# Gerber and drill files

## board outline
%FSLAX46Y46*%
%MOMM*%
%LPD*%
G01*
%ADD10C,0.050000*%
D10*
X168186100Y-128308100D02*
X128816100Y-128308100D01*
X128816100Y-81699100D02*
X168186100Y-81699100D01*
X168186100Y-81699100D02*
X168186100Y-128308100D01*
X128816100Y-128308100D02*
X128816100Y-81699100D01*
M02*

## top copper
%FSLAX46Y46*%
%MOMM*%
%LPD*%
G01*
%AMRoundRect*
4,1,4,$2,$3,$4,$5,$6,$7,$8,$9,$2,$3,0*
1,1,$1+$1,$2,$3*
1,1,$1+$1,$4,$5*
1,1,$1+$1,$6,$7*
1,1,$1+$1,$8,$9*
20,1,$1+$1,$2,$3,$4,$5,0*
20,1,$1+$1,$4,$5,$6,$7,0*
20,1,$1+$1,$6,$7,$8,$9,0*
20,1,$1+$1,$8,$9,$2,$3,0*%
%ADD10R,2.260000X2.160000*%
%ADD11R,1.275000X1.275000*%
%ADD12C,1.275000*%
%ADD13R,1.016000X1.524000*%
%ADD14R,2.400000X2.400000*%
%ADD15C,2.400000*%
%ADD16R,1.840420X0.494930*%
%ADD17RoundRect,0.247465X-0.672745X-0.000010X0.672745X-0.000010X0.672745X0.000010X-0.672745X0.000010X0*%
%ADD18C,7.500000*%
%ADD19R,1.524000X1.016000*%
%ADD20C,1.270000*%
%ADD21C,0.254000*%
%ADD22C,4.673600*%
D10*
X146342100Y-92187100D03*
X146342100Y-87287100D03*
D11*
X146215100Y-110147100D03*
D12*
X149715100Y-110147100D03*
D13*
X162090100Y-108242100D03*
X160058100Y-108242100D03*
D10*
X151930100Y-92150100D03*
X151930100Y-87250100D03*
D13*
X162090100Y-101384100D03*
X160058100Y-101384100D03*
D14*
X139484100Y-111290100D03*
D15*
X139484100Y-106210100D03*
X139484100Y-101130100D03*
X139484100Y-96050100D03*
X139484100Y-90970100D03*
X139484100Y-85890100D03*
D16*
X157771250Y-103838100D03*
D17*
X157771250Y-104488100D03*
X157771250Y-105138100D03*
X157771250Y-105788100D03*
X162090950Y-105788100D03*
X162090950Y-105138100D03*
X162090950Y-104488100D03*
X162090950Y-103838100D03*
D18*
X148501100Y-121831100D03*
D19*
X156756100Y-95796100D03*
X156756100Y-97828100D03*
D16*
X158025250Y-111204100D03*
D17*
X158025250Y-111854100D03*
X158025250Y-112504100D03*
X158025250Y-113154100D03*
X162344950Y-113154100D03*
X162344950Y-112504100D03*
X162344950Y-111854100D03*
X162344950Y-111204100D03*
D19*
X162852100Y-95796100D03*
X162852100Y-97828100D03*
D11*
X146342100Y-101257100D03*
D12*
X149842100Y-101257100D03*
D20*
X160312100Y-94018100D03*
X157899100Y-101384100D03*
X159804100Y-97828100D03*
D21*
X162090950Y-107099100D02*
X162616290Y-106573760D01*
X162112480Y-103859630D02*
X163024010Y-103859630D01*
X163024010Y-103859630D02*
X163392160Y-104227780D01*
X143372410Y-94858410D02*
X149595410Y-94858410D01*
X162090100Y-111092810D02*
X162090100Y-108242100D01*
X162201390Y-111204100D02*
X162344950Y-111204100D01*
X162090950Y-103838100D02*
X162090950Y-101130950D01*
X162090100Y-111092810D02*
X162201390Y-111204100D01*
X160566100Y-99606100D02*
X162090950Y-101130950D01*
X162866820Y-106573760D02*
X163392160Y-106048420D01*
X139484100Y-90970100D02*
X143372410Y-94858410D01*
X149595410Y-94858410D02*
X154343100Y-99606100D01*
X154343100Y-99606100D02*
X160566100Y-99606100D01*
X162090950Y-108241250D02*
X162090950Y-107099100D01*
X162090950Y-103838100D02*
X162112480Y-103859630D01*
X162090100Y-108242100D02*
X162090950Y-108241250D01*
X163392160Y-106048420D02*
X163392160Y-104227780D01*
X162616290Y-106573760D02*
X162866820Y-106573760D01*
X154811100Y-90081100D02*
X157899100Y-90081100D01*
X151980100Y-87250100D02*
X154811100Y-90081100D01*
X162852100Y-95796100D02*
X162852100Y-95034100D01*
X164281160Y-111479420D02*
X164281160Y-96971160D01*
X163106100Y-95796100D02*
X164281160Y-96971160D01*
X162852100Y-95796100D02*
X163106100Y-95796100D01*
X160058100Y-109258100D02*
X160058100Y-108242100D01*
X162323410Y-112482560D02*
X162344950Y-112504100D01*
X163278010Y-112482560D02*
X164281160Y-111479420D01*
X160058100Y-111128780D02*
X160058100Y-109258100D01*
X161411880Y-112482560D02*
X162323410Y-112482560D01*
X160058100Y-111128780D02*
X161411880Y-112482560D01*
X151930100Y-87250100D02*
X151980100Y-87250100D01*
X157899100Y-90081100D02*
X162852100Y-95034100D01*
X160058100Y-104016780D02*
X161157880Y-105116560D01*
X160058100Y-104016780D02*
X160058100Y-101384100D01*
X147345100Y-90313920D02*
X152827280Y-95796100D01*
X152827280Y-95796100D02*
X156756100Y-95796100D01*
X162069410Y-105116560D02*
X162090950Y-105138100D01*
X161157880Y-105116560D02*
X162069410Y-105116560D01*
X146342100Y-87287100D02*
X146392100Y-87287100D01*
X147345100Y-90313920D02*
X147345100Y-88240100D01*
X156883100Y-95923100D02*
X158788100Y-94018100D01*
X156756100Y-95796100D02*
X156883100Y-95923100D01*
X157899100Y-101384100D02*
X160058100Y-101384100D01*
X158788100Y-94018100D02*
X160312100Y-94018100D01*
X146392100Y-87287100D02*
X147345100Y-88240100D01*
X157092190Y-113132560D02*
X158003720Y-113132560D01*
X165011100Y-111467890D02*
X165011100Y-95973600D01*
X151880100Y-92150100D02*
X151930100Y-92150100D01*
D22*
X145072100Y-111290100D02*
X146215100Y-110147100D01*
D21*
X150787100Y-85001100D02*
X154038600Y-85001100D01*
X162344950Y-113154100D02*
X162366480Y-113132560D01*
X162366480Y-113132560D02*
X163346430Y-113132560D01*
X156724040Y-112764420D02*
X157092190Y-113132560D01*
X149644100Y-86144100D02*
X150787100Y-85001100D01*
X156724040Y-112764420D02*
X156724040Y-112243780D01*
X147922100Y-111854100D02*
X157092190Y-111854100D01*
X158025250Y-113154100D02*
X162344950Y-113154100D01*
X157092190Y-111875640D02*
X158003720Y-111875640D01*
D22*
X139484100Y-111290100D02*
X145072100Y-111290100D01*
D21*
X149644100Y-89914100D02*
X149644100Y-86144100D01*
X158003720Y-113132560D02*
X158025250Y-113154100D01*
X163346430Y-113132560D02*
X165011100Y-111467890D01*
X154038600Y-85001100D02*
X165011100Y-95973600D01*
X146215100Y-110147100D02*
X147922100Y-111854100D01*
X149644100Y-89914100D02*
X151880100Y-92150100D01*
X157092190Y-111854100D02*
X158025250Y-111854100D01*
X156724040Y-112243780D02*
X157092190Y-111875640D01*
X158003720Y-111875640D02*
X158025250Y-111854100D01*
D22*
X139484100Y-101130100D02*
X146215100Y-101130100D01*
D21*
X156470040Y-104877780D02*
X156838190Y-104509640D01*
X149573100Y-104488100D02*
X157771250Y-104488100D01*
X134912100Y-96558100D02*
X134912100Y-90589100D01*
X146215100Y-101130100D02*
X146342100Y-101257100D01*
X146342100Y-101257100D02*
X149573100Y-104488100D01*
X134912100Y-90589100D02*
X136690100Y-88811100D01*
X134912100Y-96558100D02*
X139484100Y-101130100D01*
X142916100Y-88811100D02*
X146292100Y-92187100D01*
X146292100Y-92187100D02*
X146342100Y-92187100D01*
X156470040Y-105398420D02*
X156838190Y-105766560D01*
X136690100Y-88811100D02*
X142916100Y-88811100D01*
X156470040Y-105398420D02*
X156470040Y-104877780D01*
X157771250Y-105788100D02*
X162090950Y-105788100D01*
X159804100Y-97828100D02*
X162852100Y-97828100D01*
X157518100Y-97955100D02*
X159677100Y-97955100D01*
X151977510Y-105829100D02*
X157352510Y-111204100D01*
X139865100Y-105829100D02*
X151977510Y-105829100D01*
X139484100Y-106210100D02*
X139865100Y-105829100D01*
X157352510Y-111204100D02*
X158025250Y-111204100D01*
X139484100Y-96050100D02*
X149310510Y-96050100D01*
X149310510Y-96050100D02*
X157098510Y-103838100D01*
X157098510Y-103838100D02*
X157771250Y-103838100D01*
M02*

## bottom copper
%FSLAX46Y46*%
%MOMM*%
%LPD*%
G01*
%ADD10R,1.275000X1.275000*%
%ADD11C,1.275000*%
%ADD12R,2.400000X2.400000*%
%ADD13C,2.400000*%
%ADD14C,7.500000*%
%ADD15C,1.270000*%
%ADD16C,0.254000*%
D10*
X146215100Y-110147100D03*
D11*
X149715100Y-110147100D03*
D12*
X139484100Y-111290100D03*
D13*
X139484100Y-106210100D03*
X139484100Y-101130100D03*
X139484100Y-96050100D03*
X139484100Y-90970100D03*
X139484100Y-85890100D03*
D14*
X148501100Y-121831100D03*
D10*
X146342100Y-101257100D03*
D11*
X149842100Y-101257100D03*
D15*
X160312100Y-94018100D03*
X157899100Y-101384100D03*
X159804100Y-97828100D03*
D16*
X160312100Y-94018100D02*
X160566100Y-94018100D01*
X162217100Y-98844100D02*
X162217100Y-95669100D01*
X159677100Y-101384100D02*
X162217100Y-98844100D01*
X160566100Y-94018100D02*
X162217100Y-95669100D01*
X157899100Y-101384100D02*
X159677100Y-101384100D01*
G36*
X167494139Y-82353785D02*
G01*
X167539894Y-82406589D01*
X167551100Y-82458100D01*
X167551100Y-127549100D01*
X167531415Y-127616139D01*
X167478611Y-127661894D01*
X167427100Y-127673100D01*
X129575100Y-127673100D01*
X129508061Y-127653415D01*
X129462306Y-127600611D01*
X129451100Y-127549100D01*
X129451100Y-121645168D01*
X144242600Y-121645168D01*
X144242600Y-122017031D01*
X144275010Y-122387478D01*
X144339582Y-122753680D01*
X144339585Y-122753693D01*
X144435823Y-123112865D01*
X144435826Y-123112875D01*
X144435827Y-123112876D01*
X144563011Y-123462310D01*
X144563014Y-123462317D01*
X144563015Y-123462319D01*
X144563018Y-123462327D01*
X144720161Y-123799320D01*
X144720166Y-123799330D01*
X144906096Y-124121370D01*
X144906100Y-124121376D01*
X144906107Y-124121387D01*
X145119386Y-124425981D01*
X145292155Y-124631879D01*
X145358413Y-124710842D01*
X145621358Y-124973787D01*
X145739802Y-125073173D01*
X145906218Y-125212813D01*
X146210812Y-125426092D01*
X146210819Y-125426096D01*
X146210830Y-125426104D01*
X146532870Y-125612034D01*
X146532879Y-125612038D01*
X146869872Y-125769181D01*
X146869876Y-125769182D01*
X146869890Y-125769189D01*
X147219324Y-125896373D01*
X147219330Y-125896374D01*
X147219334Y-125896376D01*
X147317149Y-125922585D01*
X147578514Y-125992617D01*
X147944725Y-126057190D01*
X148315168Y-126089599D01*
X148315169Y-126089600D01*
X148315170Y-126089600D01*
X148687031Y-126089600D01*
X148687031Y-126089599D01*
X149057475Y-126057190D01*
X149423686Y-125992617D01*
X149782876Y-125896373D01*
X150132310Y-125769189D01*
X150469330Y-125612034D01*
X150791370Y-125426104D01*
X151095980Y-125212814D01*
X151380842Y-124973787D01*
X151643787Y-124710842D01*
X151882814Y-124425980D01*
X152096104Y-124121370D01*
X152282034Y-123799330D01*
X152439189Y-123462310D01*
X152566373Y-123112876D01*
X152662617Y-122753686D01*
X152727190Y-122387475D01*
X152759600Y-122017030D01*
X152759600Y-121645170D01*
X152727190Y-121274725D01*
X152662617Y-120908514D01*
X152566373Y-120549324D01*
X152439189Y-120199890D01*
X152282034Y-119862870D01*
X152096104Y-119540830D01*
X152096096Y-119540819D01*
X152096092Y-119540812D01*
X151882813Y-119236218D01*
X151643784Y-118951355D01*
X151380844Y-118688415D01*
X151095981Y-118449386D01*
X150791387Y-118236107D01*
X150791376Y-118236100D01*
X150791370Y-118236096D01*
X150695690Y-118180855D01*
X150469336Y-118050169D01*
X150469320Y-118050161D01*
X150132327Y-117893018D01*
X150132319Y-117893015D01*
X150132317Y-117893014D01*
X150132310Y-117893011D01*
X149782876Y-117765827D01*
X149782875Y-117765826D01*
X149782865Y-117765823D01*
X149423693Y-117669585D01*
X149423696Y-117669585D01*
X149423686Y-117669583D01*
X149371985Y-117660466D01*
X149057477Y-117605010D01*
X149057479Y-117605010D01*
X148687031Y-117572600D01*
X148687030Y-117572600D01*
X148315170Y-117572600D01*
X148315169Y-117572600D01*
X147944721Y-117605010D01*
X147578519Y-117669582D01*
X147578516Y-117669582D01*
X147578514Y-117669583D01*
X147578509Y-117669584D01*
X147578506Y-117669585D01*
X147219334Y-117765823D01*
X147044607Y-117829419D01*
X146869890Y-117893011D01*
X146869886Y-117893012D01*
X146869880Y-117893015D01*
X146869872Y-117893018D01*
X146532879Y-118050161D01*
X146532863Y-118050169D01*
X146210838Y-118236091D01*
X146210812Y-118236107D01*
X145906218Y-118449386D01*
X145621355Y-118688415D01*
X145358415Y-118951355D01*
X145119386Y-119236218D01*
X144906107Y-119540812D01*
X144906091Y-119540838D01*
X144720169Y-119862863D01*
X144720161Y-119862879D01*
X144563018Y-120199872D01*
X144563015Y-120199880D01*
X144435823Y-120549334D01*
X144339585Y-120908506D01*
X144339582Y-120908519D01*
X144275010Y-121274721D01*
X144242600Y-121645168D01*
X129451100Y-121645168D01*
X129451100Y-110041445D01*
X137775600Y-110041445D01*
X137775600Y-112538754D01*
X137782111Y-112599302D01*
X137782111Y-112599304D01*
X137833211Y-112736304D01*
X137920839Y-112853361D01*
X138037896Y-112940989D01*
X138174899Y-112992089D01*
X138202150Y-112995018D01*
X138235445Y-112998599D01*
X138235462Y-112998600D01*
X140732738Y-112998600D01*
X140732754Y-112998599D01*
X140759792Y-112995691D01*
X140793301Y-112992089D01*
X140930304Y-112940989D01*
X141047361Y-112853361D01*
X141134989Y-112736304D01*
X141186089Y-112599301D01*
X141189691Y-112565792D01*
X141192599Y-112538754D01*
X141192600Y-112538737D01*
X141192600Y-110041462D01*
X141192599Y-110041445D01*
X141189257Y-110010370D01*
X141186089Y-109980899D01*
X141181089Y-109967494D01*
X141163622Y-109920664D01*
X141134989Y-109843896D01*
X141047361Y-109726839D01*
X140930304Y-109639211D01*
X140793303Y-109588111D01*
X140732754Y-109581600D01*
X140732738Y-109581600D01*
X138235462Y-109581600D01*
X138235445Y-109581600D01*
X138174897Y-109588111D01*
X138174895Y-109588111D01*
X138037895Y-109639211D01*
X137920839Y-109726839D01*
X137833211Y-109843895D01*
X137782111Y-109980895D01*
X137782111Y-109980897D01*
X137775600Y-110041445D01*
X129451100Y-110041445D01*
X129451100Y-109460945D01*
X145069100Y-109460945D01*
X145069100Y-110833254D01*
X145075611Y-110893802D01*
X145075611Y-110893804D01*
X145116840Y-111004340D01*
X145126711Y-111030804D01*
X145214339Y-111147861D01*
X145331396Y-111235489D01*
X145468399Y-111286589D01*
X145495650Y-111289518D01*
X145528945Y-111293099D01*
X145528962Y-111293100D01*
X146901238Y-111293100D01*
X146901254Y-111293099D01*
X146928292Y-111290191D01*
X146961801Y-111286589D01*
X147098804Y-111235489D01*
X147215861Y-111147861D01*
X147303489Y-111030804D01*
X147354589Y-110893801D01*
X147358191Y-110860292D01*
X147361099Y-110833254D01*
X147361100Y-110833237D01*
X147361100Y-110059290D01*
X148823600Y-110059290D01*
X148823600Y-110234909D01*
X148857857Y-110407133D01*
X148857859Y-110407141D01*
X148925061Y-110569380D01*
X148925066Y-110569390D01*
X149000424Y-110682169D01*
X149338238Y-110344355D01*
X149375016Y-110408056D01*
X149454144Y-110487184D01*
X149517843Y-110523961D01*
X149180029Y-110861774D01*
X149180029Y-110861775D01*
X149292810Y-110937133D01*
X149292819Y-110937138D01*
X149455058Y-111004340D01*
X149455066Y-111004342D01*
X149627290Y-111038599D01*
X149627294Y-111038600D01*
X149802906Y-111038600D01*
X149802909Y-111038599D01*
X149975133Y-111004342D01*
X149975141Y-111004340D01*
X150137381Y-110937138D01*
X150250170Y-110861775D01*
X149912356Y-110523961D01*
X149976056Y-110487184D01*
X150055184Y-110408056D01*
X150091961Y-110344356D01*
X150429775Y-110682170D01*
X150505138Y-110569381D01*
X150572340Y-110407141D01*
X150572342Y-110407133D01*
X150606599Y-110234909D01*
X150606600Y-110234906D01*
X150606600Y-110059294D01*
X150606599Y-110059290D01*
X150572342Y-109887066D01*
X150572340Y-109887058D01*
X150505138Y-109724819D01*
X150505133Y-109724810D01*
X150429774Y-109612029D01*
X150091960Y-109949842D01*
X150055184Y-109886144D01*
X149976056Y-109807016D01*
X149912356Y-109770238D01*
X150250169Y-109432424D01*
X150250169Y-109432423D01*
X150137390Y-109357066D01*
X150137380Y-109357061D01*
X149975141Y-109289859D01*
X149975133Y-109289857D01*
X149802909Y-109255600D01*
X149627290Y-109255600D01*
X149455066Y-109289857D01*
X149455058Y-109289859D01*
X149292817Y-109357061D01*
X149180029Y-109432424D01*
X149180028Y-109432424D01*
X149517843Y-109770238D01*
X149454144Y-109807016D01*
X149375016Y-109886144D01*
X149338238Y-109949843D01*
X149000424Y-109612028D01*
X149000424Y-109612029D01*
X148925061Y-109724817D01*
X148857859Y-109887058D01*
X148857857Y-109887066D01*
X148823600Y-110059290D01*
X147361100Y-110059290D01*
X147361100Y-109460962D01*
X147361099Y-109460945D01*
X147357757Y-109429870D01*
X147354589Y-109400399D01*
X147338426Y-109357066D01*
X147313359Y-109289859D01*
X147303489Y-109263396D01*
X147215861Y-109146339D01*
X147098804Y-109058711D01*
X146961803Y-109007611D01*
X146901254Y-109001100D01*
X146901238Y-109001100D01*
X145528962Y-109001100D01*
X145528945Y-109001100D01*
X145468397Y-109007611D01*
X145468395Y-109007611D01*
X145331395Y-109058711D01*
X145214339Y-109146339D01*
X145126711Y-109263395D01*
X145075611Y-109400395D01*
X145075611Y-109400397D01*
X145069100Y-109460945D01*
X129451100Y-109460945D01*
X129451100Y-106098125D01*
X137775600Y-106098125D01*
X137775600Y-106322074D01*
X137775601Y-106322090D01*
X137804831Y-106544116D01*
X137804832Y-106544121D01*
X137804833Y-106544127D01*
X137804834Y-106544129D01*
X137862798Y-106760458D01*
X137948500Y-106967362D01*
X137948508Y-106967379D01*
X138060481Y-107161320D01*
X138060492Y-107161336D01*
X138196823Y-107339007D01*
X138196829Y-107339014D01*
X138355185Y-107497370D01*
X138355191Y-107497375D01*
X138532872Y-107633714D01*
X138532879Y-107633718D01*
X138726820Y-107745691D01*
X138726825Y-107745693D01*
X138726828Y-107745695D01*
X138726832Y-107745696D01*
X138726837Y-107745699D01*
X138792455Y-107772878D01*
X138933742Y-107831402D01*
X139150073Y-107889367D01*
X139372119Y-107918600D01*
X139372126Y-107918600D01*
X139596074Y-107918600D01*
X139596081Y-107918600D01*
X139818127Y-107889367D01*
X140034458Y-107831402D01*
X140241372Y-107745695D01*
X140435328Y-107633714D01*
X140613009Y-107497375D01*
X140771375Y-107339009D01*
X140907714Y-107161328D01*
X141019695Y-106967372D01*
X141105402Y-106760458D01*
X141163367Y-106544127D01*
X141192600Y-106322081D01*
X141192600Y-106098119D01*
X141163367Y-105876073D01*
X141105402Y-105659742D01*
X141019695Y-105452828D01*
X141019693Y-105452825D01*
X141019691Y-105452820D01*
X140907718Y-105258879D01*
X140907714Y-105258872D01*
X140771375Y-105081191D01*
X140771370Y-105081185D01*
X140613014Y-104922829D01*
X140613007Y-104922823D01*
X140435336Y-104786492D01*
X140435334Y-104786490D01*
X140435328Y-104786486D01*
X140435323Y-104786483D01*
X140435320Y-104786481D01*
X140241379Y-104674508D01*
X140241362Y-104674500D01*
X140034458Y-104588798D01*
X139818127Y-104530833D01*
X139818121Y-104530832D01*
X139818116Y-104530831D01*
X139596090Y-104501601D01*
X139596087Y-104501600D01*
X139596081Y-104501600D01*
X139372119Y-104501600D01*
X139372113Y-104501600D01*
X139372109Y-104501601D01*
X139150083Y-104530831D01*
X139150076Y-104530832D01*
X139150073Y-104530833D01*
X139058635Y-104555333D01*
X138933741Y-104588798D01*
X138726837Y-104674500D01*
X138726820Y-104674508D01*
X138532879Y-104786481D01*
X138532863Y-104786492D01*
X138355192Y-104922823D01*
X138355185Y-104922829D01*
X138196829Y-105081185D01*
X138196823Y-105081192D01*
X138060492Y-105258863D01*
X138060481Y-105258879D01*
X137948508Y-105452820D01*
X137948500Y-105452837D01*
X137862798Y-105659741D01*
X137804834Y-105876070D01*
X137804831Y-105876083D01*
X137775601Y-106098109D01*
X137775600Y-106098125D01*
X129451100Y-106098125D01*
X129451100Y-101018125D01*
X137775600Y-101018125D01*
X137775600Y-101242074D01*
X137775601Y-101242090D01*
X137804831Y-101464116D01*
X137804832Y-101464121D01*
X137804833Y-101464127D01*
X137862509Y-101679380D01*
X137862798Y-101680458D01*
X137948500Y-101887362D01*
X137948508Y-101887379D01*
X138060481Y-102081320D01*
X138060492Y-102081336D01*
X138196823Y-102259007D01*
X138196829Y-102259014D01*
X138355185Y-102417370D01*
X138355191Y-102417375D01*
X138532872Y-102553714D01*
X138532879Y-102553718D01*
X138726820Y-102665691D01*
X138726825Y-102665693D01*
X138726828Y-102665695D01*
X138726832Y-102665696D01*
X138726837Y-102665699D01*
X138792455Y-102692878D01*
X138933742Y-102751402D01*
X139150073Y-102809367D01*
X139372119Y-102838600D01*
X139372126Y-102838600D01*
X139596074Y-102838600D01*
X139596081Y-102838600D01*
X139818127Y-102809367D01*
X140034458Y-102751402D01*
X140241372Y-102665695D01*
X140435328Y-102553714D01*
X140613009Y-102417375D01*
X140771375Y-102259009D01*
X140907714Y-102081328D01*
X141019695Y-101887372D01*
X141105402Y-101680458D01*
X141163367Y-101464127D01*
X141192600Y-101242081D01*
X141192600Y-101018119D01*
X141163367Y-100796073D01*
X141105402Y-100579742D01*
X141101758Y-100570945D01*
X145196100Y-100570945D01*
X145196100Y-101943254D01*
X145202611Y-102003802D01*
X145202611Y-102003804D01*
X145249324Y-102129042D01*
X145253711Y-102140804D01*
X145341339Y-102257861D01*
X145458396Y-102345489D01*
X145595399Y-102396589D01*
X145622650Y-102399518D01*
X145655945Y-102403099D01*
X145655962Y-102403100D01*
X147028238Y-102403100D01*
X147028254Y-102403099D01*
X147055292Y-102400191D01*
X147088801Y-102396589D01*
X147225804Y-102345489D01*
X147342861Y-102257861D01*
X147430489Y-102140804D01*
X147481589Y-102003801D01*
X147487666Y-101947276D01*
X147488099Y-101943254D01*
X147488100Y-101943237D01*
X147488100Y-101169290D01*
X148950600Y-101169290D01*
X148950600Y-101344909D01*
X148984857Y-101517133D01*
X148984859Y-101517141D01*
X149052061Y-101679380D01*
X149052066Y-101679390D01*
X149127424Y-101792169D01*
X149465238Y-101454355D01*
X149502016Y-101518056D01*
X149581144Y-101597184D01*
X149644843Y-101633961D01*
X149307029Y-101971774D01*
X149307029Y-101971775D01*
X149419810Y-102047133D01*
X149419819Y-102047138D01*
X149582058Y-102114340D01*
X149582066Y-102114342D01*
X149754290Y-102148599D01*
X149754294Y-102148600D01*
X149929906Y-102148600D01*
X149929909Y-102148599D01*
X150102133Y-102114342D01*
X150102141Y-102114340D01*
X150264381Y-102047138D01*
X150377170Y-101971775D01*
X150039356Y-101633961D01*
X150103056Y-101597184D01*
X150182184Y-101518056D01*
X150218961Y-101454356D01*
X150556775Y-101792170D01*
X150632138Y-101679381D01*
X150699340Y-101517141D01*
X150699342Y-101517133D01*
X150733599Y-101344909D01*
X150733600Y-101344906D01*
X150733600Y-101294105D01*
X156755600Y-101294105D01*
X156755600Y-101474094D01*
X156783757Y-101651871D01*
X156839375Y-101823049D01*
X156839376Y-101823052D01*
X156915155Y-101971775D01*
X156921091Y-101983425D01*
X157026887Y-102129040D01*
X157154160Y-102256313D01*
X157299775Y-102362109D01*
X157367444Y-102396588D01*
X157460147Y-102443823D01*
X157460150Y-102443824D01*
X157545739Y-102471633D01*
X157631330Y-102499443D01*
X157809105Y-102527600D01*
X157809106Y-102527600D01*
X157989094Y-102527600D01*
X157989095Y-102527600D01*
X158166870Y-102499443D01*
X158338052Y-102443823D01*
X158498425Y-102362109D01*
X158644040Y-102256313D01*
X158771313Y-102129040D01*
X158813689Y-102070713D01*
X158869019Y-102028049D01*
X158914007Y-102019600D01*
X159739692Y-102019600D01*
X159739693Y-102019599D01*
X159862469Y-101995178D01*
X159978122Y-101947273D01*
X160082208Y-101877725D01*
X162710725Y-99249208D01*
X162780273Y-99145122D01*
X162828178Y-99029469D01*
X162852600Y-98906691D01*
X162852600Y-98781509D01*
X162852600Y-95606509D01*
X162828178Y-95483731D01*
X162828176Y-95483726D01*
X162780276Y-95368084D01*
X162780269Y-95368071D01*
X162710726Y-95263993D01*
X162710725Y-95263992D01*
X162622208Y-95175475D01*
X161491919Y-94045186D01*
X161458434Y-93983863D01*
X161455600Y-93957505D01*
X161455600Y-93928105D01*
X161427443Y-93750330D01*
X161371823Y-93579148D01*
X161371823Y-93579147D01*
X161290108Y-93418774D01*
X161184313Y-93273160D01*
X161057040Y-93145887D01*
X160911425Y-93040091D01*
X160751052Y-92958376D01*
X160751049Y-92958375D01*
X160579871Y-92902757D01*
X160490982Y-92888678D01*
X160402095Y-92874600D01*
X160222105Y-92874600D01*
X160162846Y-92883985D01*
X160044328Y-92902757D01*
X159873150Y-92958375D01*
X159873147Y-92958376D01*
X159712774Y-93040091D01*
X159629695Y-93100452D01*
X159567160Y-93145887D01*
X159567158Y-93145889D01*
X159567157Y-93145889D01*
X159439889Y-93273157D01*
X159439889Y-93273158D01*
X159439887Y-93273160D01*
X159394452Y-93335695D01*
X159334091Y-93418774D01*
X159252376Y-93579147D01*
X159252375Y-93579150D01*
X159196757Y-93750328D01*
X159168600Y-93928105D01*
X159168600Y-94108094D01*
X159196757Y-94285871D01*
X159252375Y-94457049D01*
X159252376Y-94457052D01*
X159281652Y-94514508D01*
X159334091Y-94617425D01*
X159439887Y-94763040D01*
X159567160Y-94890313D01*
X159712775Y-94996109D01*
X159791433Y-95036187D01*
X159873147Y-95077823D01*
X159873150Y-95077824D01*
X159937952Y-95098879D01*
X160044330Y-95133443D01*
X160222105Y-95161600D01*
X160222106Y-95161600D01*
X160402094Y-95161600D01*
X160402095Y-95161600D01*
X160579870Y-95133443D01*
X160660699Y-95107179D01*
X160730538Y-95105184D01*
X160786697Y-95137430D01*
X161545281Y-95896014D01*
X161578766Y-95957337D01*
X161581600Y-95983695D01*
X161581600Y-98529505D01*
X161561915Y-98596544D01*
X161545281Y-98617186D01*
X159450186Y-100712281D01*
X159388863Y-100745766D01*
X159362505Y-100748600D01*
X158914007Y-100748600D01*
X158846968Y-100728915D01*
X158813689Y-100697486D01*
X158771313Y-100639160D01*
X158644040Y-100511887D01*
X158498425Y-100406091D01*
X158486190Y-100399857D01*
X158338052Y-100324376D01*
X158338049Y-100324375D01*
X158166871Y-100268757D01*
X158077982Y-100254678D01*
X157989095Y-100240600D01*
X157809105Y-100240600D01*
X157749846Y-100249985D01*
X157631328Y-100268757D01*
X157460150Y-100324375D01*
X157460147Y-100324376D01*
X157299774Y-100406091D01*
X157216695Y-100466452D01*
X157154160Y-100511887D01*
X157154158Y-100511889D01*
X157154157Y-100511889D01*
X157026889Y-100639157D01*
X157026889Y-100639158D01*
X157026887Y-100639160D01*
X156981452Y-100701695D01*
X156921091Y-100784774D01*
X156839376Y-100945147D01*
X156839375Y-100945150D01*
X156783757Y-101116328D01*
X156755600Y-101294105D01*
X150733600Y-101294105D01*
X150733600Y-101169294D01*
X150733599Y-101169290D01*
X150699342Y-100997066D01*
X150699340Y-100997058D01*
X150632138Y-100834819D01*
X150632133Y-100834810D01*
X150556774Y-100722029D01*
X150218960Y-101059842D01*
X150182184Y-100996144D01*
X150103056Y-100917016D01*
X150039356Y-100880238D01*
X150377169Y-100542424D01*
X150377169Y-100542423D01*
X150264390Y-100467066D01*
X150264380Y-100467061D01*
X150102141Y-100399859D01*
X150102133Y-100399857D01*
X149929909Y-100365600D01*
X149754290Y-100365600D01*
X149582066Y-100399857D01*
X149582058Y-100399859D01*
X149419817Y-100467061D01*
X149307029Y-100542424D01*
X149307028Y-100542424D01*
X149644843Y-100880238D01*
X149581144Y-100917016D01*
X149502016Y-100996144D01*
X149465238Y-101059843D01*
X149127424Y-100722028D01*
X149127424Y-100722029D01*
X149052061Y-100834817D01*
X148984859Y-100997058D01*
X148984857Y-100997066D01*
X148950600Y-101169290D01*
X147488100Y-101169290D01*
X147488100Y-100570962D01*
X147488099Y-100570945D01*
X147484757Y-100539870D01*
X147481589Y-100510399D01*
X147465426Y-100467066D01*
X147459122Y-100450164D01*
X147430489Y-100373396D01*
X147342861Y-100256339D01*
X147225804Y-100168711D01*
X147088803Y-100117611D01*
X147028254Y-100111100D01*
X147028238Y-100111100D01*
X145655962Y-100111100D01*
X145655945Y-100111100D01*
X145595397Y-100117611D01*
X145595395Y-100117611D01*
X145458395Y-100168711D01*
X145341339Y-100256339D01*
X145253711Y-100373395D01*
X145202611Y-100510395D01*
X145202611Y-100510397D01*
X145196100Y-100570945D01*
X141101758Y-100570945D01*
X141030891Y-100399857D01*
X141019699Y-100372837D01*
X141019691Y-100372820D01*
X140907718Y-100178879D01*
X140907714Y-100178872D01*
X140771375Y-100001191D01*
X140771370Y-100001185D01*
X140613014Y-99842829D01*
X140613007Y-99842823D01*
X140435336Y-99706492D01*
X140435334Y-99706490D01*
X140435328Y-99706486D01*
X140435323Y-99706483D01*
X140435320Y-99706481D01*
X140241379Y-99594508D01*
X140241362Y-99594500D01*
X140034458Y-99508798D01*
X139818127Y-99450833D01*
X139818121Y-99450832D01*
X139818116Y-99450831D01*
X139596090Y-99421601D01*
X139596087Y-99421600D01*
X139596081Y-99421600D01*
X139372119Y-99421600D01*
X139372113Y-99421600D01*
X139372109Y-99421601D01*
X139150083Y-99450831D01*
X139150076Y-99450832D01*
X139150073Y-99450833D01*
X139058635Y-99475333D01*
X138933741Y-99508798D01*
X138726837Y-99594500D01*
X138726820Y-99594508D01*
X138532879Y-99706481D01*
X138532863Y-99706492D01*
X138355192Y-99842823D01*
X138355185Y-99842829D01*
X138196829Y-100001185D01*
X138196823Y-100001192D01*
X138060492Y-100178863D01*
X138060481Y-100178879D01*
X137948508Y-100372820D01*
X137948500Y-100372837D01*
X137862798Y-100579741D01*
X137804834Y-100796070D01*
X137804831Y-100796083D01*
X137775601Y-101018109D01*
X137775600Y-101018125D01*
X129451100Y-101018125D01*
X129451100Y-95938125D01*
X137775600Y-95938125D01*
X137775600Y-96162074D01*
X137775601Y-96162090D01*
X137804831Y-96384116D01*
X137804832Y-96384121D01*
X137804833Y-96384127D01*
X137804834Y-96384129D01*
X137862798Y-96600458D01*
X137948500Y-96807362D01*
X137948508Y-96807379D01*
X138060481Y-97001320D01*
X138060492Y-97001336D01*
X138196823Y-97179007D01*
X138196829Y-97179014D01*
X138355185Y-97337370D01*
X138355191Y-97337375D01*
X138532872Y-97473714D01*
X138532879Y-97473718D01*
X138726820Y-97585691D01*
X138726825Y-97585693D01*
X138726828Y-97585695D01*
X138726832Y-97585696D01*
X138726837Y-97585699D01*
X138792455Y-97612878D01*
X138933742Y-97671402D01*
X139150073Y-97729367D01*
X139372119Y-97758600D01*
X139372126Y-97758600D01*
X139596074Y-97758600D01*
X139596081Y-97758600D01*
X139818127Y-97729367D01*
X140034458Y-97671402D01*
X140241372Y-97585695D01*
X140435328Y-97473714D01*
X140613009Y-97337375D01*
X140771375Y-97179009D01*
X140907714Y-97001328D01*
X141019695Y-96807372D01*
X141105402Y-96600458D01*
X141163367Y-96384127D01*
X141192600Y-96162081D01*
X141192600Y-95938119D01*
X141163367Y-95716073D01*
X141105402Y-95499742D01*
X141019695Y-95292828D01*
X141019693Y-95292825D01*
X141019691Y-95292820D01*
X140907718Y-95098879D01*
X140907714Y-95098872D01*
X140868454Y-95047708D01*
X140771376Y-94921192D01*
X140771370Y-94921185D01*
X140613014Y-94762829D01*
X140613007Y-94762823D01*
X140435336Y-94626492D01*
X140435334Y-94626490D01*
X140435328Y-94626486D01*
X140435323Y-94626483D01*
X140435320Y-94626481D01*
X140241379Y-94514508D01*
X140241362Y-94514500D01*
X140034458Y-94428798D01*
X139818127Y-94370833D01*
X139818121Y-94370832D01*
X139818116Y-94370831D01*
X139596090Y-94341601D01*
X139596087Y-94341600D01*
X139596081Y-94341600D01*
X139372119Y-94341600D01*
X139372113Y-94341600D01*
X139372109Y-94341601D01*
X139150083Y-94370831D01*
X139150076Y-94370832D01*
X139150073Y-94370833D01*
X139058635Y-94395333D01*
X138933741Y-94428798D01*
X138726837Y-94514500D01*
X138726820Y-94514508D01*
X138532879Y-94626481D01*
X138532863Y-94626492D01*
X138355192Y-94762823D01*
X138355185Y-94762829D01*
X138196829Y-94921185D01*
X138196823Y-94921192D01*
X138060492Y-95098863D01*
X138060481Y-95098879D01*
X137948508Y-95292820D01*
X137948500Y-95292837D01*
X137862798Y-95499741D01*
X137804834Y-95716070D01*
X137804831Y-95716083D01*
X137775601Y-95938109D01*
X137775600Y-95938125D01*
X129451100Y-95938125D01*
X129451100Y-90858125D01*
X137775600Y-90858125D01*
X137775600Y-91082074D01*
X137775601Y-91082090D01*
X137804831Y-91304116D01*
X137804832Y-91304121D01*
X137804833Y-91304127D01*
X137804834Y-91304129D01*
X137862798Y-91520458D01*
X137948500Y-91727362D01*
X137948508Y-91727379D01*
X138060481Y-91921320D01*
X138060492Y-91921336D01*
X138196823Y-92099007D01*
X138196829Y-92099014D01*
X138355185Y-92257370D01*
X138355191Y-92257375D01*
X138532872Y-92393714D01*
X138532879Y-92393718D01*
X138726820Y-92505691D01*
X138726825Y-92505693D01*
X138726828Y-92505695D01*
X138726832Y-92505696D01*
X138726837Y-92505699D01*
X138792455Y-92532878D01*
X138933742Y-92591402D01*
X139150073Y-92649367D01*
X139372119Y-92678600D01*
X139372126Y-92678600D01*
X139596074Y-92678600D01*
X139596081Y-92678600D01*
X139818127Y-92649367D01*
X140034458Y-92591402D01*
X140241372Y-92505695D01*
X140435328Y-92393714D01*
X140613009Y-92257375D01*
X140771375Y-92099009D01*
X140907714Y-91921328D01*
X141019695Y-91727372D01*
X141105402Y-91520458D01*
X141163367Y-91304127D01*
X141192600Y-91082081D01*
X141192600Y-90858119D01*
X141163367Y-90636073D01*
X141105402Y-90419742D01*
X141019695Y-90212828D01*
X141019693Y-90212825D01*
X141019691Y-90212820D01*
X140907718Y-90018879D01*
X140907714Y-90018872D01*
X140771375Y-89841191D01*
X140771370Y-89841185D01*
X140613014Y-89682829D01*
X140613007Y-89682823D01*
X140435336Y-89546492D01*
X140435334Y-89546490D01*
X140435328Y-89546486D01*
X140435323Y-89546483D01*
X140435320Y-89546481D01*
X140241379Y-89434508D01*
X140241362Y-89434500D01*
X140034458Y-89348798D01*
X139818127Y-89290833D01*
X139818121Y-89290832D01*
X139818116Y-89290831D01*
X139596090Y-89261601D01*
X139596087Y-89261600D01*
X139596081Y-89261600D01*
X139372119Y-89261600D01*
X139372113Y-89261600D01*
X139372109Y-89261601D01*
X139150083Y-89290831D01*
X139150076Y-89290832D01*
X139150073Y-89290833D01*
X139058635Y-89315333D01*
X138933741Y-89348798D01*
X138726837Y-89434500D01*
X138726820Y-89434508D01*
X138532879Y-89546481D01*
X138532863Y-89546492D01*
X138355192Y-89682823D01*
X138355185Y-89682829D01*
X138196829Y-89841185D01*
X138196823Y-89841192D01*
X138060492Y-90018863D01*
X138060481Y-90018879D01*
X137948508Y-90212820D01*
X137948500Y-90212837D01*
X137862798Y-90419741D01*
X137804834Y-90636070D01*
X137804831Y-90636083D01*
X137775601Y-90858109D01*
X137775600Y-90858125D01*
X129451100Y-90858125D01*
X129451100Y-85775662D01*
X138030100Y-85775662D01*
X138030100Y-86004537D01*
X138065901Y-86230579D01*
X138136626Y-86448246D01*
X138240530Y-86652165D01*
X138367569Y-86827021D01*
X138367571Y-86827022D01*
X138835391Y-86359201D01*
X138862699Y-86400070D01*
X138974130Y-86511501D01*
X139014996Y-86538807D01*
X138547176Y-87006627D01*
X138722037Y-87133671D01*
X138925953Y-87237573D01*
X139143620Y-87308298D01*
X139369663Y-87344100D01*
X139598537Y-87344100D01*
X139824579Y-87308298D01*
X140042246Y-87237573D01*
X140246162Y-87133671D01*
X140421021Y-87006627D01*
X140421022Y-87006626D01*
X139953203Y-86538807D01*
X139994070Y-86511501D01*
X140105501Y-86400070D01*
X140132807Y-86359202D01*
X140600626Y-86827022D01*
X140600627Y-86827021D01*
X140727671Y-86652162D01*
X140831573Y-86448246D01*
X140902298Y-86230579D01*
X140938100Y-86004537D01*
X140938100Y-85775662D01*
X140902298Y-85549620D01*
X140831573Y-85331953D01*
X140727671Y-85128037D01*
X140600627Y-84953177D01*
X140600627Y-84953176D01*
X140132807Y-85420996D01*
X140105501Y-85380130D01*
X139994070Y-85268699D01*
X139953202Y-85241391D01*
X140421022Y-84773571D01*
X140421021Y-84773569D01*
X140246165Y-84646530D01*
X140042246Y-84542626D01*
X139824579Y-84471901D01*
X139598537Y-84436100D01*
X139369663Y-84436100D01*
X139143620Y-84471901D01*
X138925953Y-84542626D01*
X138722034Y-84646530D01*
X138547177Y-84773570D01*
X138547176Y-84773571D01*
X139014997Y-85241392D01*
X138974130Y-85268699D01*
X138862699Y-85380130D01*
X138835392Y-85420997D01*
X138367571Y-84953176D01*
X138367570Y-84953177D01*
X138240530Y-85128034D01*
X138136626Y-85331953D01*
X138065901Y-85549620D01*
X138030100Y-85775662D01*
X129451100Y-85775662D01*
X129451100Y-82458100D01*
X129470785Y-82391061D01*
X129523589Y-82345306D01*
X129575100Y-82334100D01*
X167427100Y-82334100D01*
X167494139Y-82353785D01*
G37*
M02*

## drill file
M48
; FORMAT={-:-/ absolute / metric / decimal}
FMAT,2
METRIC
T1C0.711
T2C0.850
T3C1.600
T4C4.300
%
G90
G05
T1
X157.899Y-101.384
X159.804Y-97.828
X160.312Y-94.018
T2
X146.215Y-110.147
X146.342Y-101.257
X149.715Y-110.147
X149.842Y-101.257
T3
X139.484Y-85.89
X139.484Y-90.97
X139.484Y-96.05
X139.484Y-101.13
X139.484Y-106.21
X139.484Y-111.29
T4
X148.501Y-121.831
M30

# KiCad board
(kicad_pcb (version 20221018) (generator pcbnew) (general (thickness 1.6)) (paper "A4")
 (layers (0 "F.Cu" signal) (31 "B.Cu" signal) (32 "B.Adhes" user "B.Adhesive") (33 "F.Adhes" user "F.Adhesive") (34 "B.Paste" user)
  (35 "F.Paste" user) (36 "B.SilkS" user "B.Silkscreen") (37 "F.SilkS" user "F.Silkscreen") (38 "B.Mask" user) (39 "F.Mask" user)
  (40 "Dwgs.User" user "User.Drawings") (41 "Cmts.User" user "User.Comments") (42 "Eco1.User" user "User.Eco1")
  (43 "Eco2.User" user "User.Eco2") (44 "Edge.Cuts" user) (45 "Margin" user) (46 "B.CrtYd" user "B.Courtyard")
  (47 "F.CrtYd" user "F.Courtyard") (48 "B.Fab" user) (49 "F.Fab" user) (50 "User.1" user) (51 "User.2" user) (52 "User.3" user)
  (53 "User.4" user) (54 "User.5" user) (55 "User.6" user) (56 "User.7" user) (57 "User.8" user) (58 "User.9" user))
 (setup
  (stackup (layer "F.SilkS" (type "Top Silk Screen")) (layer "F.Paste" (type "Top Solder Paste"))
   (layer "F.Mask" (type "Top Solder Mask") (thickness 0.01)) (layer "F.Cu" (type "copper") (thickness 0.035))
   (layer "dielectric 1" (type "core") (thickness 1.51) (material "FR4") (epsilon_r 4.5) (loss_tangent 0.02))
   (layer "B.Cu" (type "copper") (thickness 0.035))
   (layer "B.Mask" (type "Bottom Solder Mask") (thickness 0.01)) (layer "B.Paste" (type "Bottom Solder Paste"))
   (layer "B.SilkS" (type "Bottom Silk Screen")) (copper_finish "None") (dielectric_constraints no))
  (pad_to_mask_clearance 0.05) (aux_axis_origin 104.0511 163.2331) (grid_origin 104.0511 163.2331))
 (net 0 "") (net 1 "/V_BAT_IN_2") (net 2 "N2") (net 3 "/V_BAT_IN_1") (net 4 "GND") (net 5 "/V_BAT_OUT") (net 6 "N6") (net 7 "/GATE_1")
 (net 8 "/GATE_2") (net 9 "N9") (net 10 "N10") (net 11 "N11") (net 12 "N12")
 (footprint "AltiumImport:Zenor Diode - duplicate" (layer "F.Cu") (at 146.3421 89.7371 90)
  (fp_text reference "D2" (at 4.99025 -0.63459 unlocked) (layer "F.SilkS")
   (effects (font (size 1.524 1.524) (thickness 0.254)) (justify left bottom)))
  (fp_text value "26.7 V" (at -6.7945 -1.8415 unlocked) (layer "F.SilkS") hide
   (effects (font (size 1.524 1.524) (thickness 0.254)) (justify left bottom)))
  (pad "A" smd rect (at -2.45 0 90) (size 2.16 2.26) (layers "F.Cu" "F.Paste" "F.Mask") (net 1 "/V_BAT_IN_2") (thermal_bridge_angle 45))
  (pad "K" smd rect (at 2.45 0 90) (size 2.16 2.26) (layers "F.Cu" "F.Paste" "F.Mask") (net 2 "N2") (thermal_bridge_angle 45)))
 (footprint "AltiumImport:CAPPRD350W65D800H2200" (layer "F.Cu") (at 146.2151 110.1471)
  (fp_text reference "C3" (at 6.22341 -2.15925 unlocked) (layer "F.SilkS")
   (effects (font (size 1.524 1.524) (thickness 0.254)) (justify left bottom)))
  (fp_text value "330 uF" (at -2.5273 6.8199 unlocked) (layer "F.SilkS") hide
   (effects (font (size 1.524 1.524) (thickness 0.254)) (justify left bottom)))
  (pad "1" thru_hole rect (at 0 0) (size 1.275 1.275) (drill 0.85) (layers "*.Cu" "*.Mask") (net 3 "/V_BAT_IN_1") (thermal_bridge_angle 45))
  (pad "2" thru_hole circle (at 3.5 0) (size 1.275 1.275) (drill 0.85) (layers "*.Cu" "*.Mask") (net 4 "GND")))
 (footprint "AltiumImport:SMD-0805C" (layer "F.Cu") (at 161.0741 108.2421 -90)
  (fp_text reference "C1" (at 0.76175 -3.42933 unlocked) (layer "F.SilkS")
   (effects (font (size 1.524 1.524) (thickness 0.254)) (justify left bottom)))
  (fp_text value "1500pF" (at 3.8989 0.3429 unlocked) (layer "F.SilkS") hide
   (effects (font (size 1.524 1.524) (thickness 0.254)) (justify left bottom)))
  (pad "1" smd rect (at 0 -1.016 180) (size 1.016 1.524) (layers "F.Cu" "F.Paste" "F.Mask") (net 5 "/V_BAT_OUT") (thermal_bridge_angle 45))
  (pad "2" smd rect (at 0 1.016 180) (size 1.016 1.524) (layers "F.Cu" "F.Paste" "F.Mask") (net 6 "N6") (thermal_bridge_angle 45)))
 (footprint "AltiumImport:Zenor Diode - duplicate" (layer "F.Cu") (at 151.9301 89.7001 90)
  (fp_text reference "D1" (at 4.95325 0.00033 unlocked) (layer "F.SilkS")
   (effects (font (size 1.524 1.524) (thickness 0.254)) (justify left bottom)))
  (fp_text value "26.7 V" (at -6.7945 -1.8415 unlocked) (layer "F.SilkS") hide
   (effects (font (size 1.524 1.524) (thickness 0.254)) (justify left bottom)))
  (pad "A" smd rect (at -2.45 0 90) (size 2.16 2.26) (layers "F.Cu" "F.Paste" "F.Mask") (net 3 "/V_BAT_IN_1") (thermal_bridge_angle 45))
  (pad "K" smd rect (at 2.45 0 90) (size 2.16 2.26) (layers "F.Cu" "F.Paste" "F.Mask") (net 6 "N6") (thermal_bridge_angle 45)))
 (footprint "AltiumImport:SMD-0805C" (layer "F.Cu") (at 161.0741 101.3841 -90)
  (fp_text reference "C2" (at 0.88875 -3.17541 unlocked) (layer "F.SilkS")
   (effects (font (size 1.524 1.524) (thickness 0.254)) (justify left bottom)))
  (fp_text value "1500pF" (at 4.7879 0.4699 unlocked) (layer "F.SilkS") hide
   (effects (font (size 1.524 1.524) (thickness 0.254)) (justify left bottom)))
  (pad "1" smd rect (at 0 -1.016 180) (size 1.016 1.524) (layers "F.Cu" "F.Paste" "F.Mask") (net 5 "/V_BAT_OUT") (thermal_bridge_angle 45))
  (pad "2" smd rect (at 0 1.016 180) (size 1.016 1.524) (layers "F.Cu" "F.Paste" "F.Mask") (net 2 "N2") (thermal_bridge_angle 45)))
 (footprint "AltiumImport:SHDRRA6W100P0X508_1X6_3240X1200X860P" (layer "F.Cu") (at 139.4841 111.2901 90)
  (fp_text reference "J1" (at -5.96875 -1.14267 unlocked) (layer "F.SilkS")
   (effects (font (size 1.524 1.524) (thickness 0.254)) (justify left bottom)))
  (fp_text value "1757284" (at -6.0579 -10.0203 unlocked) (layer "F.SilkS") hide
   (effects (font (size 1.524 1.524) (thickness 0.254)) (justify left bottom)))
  (pad "1" thru_hole rect (at 0 0 90) (size 2.4 2.4) (drill 1.6) (layers "*.Cu" "*.Mask") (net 3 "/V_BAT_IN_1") (thermal_bridge_angle 45))
  (pad "2" thru_hole circle (at 5.08 0 90) (size 2.4 2.4) (drill 1.6) (layers "*.Cu" "*.Mask") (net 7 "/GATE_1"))
  (pad "3" thru_hole circle (at 10.16 0 90) (size 2.4 2.4) (drill 1.6) (layers "*.Cu" "*.Mask") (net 1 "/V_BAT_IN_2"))
  (pad "4" thru_hole circle (at 15.24 0 90) (size 2.4 2.4) (drill 1.6) (layers "*.Cu" "*.Mask") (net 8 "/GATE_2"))
  (pad "5" thru_hole circle (at 20.32 0 90) (size 2.4 2.4) (drill 1.6) (layers "*.Cu" "*.Mask") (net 5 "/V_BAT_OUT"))
  (pad "6" thru_hole circle (at 25.4 0 90) (size 2.4 2.4) (drill 1.6) (layers "*.Cu" "*.Mask") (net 4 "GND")))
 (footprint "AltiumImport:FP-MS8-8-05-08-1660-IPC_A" (layer "F.Cu") (at 159.9311 104.8131)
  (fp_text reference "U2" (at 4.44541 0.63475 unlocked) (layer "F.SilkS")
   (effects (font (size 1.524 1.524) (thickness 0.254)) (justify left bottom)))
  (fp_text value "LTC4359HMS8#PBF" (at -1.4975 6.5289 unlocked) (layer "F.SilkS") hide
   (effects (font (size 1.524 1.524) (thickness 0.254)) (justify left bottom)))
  (pad "1" smd rect (at -2.15985 -0.975) (size 1.84042 0.49493) (layers "F.Cu" "F.Paste" "F.Mask") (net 8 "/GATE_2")
   (thermal_bridge_angle 45))
  (pad "2" smd roundrect (at -2.15985 -0.325) (size 1.84042 0.49493) (layers "F.Cu" "F.Paste" "F.Mask") (roundrect_rratio 0.5)
   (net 1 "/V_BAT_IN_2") (thermal_bridge_angle 45))
  (pad "3" smd roundrect (at -2.15985 0.325) (size 1.84042 0.49493) (layers "F.Cu" "F.Paste" "F.Mask") (roundrect_rratio 0.5) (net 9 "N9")
   (thermal_bridge_angle 45))
  (pad "4" smd roundrect (at -2.15985 0.975) (size 1.84042 0.49493) (layers "F.Cu" "F.Paste" "F.Mask") (roundrect_rratio 0.5)
   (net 1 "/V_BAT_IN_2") (thermal_bridge_angle 45))
  (pad "5" smd roundrect (at 2.15985 0.975) (size 1.84042 0.49493) (layers "F.Cu" "F.Paste" "F.Mask") (roundrect_rratio 0.5)
   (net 1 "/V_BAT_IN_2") (thermal_bridge_angle 45))
  (pad "6" smd roundrect (at 2.15985 0.325) (size 1.84042 0.49493) (layers "F.Cu" "F.Paste" "F.Mask") (roundrect_rratio 0.5) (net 2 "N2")
   (thermal_bridge_angle 45))
  (pad "7" smd roundrect (at 2.15985 -0.325) (size 1.84042 0.49493) (layers "F.Cu" "F.Paste" "F.Mask") (roundrect_rratio 0.5) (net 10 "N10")
   (thermal_bridge_angle 45))
  (pad "8" smd roundrect (at 2.15985 -0.975) (size 1.84042 0.49493) (layers "F.Cu" "F.Paste" "F.Mask") (roundrect_rratio 0.5)
   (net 5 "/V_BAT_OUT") (thermal_bridge_angle 45)))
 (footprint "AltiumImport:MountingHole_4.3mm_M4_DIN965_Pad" (layer "F.Cu") (at 148.5011 121.8311)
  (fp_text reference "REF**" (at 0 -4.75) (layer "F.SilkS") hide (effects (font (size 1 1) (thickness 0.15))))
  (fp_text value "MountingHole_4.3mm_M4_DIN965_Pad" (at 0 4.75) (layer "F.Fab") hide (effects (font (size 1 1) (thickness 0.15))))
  (pad "1" thru_hole circle (at 0 0) (size 7.5 7.5) (drill 4.3) (layers "*.Cu" "*.Mask")))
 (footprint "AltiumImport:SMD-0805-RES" (layer "F.Cu") (at 156.7561 96.8121)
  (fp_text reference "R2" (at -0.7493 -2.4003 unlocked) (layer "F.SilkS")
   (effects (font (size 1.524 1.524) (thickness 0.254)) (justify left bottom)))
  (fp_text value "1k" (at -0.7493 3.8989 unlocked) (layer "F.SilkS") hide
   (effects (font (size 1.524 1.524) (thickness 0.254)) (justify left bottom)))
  (pad "1" smd rect (at 0 -1.016 270) (size 1.016 1.524) (layers "F.Cu" "F.Paste" "F.Mask") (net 2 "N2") (thermal_bridge_angle 45))
  (pad "2" smd rect (at 0 1.016 270) (size 1.016 1.524) (layers "F.Cu" "F.Paste" "F.Mask") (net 4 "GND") (thermal_bridge_angle 45)))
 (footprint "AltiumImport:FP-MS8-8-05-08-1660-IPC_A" (layer "F.Cu") (at 160.1851 112.1791)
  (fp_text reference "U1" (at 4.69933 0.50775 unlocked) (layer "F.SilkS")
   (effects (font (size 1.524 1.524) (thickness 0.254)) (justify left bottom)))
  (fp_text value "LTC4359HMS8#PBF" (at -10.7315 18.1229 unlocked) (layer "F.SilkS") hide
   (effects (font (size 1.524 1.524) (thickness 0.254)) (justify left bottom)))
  (pad "1" smd rect (at -2.15985 -0.975) (size 1.84042 0.49493) (layers "F.Cu" "F.Paste" "F.Mask") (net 7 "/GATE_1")
   (thermal_bridge_angle 45))
  (pad "2" smd roundrect (at -2.15985 -0.325) (size 1.84042 0.49493) (layers "F.Cu" "F.Paste" "F.Mask") (roundrect_rratio 0.5)
   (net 3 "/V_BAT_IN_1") (thermal_bridge_angle 45))
  (pad "3" smd roundrect (at -2.15985 0.325) (size 1.84042 0.49493) (layers "F.Cu" "F.Paste" "F.Mask") (roundrect_rratio 0.5) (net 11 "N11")
   (thermal_bridge_angle 45))
  (pad "4" smd roundrect (at -2.15985 0.975) (size 1.84042 0.49493) (layers "F.Cu" "F.Paste" "F.Mask") (roundrect_rratio 0.5)
   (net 3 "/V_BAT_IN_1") (thermal_bridge_angle 45))
  (pad "5" smd roundrect (at 2.15985 0.975) (size 1.84042 0.49493) (layers "F.Cu" "F.Paste" "F.Mask") (roundrect_rratio 0.5)
   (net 3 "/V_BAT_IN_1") (thermal_bridge_angle 45))
  (pad "6" smd roundrect (at 2.15985 0.325) (size 1.84042 0.49493) (layers "F.Cu" "F.Paste" "F.Mask") (roundrect_rratio 0.5) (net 6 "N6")
   (thermal_bridge_angle 45))
  (pad "7" smd roundrect (at 2.15985 -0.325) (size 1.84042 0.49493) (layers "F.Cu" "F.Paste" "F.Mask") (roundrect_rratio 0.5) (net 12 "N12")
   (thermal_bridge_angle 45))
  (pad "8" smd roundrect (at 2.15985 -0.975) (size 1.84042 0.49493) (layers "F.Cu" "F.Paste" "F.Mask") (roundrect_rratio 0.5)
   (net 5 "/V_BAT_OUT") (thermal_bridge_angle 45)))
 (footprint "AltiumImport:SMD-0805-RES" (layer "F.Cu") (at 162.8521 96.8121)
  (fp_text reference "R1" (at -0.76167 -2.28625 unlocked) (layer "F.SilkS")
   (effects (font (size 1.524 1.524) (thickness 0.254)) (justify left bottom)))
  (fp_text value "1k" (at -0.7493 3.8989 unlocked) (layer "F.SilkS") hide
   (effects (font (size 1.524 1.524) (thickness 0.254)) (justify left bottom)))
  (pad "1" smd rect (at 0 -1.016 270) (size 1.016 1.524) (layers "F.Cu" "F.Paste" "F.Mask") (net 6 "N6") (thermal_bridge_angle 45))
  (pad "2" smd rect (at 0 1.016 270) (size 1.016 1.524) (layers "F.Cu" "F.Paste" "F.Mask") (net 4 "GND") (thermal_bridge_angle 45)))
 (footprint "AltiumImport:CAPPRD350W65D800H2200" (layer "F.Cu") (at 146.3421 101.2571)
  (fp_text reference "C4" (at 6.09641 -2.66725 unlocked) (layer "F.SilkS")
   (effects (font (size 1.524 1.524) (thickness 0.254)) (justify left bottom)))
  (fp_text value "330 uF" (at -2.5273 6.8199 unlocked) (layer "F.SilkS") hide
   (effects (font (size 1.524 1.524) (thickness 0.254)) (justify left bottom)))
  (pad "1" thru_hole rect (at 0 0) (size 1.275 1.275) (drill 0.85) (layers "*.Cu" "*.Mask") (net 1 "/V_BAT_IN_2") (thermal_bridge_angle 45))
  (pad "2" thru_hole circle (at 3.5 0) (size 1.275 1.275) (drill 0.85) (layers "*.Cu" "*.Mask") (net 4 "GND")))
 (gr_line (start 168.1861 128.3081) (end 128.8161 128.3081) (stroke (width 0.05) (type solid)) (layer "Edge.Cuts"))
 (gr_line (start 128.8161 81.6991) (end 168.1861 81.6991) (stroke (width 0.05) (type solid)) (layer "Edge.Cuts"))
 (gr_line (start 168.1861 81.6991) (end 168.1861 128.3081) (stroke (width 0.05) (type solid)) (layer "Edge.Cuts"))
 (gr_line (start 128.8161 128.3081) (end 128.8161 81.6991) (stroke (width 0.05) (type solid)) (layer "Edge.Cuts"))
 (segment (start 162.09095 107.0991) (end 162.61629 106.57376) (width 0.254) (layer "F.Cu") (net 5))
 (segment (start 162.11248 103.85963) (end 163.02401 103.85963) (width 0.254) (layer "F.Cu") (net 5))
 (segment (start 163.02401 103.85963) (end 163.39216 104.22778) (width 0.254) (layer "F.Cu") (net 5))
 (segment (start 143.37241 94.85841) (end 149.59541 94.85841) (width 0.254) (layer "F.Cu") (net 5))
 (segment (start 162.0901 111.09281) (end 162.0901 108.2421) (width 0.254) (layer "F.Cu") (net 5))
 (segment (start 162.20139 111.2041) (end 162.34495 111.2041) (width 0.254) (layer "F.Cu") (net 5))
 (segment (start 162.09095 103.8381) (end 162.09095 101.13095) (width 0.254) (layer "F.Cu") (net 5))
 (segment (start 162.0901 111.09281) (end 162.20139 111.2041) (width 0.254) (layer "F.Cu") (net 5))
 (segment (start 160.5661 99.6061) (end 162.09095 101.13095) (width 0.254) (layer "F.Cu") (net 5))
 (segment (start 162.86682 106.57376) (end 163.39216 106.04842) (width 0.254) (layer "F.Cu") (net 5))
 (segment (start 139.4841 90.9701) (end 143.37241 94.85841) (width 0.254) (layer "F.Cu") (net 5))
 (segment (start 149.59541 94.85841) (end 154.3431 99.6061) (width 0.254) (layer "F.Cu") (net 5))
 (segment (start 154.3431 99.6061) (end 160.5661 99.6061) (width 0.254) (layer "F.Cu") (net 5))
 (segment (start 162.09095 108.24125) (end 162.09095 107.0991) (width 0.254) (layer "F.Cu") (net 5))
 (segment (start 162.09095 103.8381) (end 162.11248 103.85963) (width 0.254) (layer "F.Cu") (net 5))
 (segment (start 162.0901 108.2421) (end 162.09095 108.24125) (width 0.254) (layer "F.Cu") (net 5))
 (segment (start 163.39216 106.04842) (end 163.39216 104.22778) (width 0.254) (layer "F.Cu") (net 5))
 (segment (start 162.61629 106.57376) (end 162.86682 106.57376) (width 0.254) (layer "F.Cu") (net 5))
 (segment (start 154.8111 90.0811) (end 157.8991 90.0811) (width 0.254) (layer "F.Cu") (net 6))
 (segment (start 151.9801 87.2501) (end 154.8111 90.0811) (width 0.254) (layer "F.Cu") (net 6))
 (segment (start 162.8521 95.7961) (end 162.8521 95.0341) (width 0.254) (layer "F.Cu") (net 6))
 (segment (start 164.28116 111.47942) (end 164.28116 96.97116) (width 0.254) (layer "F.Cu") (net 6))
 (segment (start 163.1061 95.7961) (end 164.28116 96.97116) (width 0.254) (layer "F.Cu") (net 6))
 (segment (start 162.8521 95.7961) (end 163.1061 95.7961) (width 0.254) (layer "F.Cu") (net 6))
 (segment (start 160.0581 109.2581) (end 160.0581 108.2421) (width 0.254) (layer "F.Cu") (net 6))
 (segment (start 162.32341 112.48256) (end 162.34495 112.5041) (width 0.254) (layer "F.Cu") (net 6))
 (segment (start 163.27801 112.48256) (end 164.28116 111.47942) (width 0.254) (layer "F.Cu") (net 6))
 (segment (start 160.0581 111.12878) (end 160.0581 109.2581) (width 0.254) (layer "F.Cu") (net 6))
 (segment (start 161.41188 112.48256) (end 162.32341 112.48256) (width 0.254) (layer "F.Cu") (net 6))
 (segment (start 160.0581 111.12878) (end 161.41188 112.48256) (width 0.254) (layer "F.Cu") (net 6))
 (segment (start 151.9301 87.2501) (end 151.9801 87.2501) (width 0.254) (layer "F.Cu") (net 6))
 (segment (start 157.8991 90.0811) (end 162.8521 95.0341) (width 0.254) (layer "F.Cu") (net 6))
 (segment (start 160.0581 104.01678) (end 161.15788 105.11656) (width 0.254) (layer "F.Cu") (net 2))
 (segment (start 160.0581 104.01678) (end 160.0581 101.3841) (width 0.254) (layer "F.Cu") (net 2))
 (segment (start 147.3451 90.31392) (end 152.82728 95.7961) (width 0.254) (layer "F.Cu") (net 2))
 (segment (start 152.82728 95.7961) (end 156.7561 95.7961) (width 0.254) (layer "F.Cu") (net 2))
 (segment (start 162.06941 105.11656) (end 162.09095 105.1381) (width 0.254) (layer "F.Cu") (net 2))
 (segment (start 161.15788 105.11656) (end 162.06941 105.11656) (width 0.254) (layer "F.Cu") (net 2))
 (segment (start 146.3421 87.2871) (end 146.3921 87.2871) (width 0.254) (layer "F.Cu") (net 2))
 (segment (start 147.3451 90.31392) (end 147.3451 88.2401) (width 0.254) (layer "F.Cu") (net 2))
 (segment (start 156.8831 95.9231) (end 158.7881 94.0181) (width 0.254) (layer "F.Cu") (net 2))
 (segment (start 156.7561 95.7961) (end 156.8831 95.9231) (width 0.254) (layer "F.Cu") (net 2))
 (segment (start 157.8991 101.3841) (end 160.0581 101.3841) (width 0.254) (layer "F.Cu") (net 2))
 (segment (start 158.7881 94.0181) (end 160.3121 94.0181) (width 0.254) (layer "F.Cu") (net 2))
 (segment (start 146.3921 87.2871) (end 147.3451 88.2401) (width 0.254) (layer "F.Cu") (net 2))
 (via (at 160.3121 94.0181) (size 1.27) (drill 0.7112) (layers "F.Cu" "B.Cu") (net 2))
 (via (at 157.8991 101.3841) (size 1.27) (drill 0.7112) (layers "F.Cu" "B.Cu") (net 2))
 (segment (start 160.3121 94.0181) (end 160.5661 94.0181) (width 0.254) (layer "B.Cu") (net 2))
 (segment (start 162.2171 98.8441) (end 162.2171 95.6691) (width 0.254) (layer "B.Cu") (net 2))
 (segment (start 159.6771 101.3841) (end 162.2171 98.8441) (width 0.254) (layer "B.Cu") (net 2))
 (segment (start 160.5661 94.0181) (end 162.2171 95.6691) (width 0.254) (layer "B.Cu") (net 2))
 (segment (start 157.8991 101.3841) (end 159.6771 101.3841) (width 0.254) (layer "B.Cu") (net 2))
 (segment (start 157.09219 113.13256) (end 158.00372 113.13256) (width 0.254) (layer "F.Cu") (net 3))
 (segment (start 165.0111 111.46789) (end 165.0111 95.9736) (width 0.254) (layer "F.Cu") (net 3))
 (segment (start 151.8801 92.1501) (end 151.9301 92.1501) (width 0.254) (layer "F.Cu") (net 3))
 (segment (start 145.0721 111.2901) (end 146.2151 110.1471) (width 4.6736) (layer "F.Cu") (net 3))
 (segment (start 150.7871 85.0011) (end 154.0386 85.0011) (width 0.254) (layer "F.Cu") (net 3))
 (segment (start 162.34495 113.1541) (end 162.36648 113.13256) (width 0.254) (layer "F.Cu") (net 3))
 (segment (start 162.36648 113.13256) (end 163.34643 113.13256) (width 0.254) (layer "F.Cu") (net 3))
 (segment (start 156.72404 112.76442) (end 157.09219 113.13256) (width 0.254) (layer "F.Cu") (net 3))
 (segment (start 149.6441 86.1441) (end 150.7871 85.0011) (width 0.254) (layer "F.Cu") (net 3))
 (segment (start 156.72404 112.76442) (end 156.72404 112.24378) (width 0.254) (layer "F.Cu") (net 3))
 (segment (start 147.9221 111.8541) (end 157.09219 111.8541) (width 0.254) (layer "F.Cu") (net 3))
 (segment (start 158.02525 113.1541) (end 162.34495 113.1541) (width 0.254) (layer "F.Cu") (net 3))
 (segment (start 157.09219 111.87564) (end 158.00372 111.87564) (width 0.254) (layer "F.Cu") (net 3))
 (segment (start 139.4841 111.2901) (end 145.0721 111.2901) (width 4.6736) (layer "F.Cu") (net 3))
 (segment (start 149.6441 89.9141) (end 149.6441 86.1441) (width 0.254) (layer "F.Cu") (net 3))
 (segment (start 158.00372 113.13256) (end 158.02525 113.1541) (width 0.254) (layer "F.Cu") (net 3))
 (segment (start 163.34643 113.13256) (end 165.0111 111.46789) (width 0.254) (layer "F.Cu") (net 3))
 (segment (start 154.0386 85.0011) (end 165.0111 95.9736) (width 0.254) (layer "F.Cu") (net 3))
 (segment (start 146.2151 110.1471) (end 147.9221 111.8541) (width 0.254) (layer "F.Cu") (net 3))
 (segment (start 149.6441 89.9141) (end 151.8801 92.1501) (width 0.254) (layer "F.Cu") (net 3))
 (segment (start 157.09219 111.8541) (end 158.02525 111.8541) (width 0.254) (layer "F.Cu") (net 3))
 (segment (start 156.72404 112.24378) (end 157.09219 111.87564) (width 0.254) (layer "F.Cu") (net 3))
 (segment (start 158.00372 111.87564) (end 158.02525 111.8541) (width 0.254) (layer "F.Cu") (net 3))
 (segment (start 139.4841 101.1301) (end 146.2151 101.1301) (width 4.6736) (layer "F.Cu") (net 1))
 (segment (start 156.47004 104.87778) (end 156.83819 104.50964) (width 0.254) (layer "F.Cu") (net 1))
 (segment (start 149.5731 104.4881) (end 157.77125 104.4881) (width 0.254) (layer "F.Cu") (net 1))
 (segment (start 134.9121 96.5581) (end 134.9121 90.5891) (width 0.254) (layer "F.Cu") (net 1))
 (segment (start 146.2151 101.1301) (end 146.3421 101.2571) (width 0.254) (layer "F.Cu") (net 1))
 (segment (start 146.3421 101.2571) (end 149.5731 104.4881) (width 0.254) (layer "F.Cu") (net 1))
 (segment (start 134.9121 90.5891) (end 136.6901 88.8111) (width 0.254) (layer "F.Cu") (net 1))
 (segment (start 134.9121 96.5581) (end 139.4841 101.1301) (width 0.254) (layer "F.Cu") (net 1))
 (segment (start 142.9161 88.8111) (end 146.2921 92.1871) (width 0.254) (layer "F.Cu") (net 1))
 (segment (start 146.2921 92.1871) (end 146.3421 92.1871) (width 0.254) (layer "F.Cu") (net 1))
 (segment (start 156.47004 105.39842) (end 156.83819 105.76656) (width 0.254) (layer "F.Cu") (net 1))
 (segment (start 136.6901 88.8111) (end 142.9161 88.8111) (width 0.254) (layer "F.Cu") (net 1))
 (segment (start 156.47004 105.39842) (end 156.47004 104.87778) (width 0.254) (layer "F.Cu") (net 1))
 (segment (start 157.77125 105.7881) (end 162.09095 105.7881) (width 0.254) (layer "F.Cu") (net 1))
 (segment (start 159.8041 97.8281) (end 162.8521 97.8281) (width 0.254) (layer "F.Cu") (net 4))
 (segment (start 157.5181 97.9551) (end 159.6771 97.9551) (width 0.254) (layer "F.Cu") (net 4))
 (via (at 159.8041 97.8281) (size 1.27) (drill 0.7112) (layers "F.Cu" "B.Cu") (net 4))
 (segment (start 151.97751 105.8291) (end 157.35251 111.2041) (width 0.254) (layer "F.Cu") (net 7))
 (segment (start 139.8651 105.8291) (end 151.97751 105.8291) (width 0.254) (layer "F.Cu") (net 7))
 (segment (start 139.4841 106.2101) (end 139.8651 105.8291) (width 0.254) (layer "F.Cu") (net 7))
 (segment (start 157.35251 111.2041) (end 158.02525 111.2041) (width 0.254) (layer "F.Cu") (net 7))
 (segment (start 139.4841 96.0501) (end 149.31051 96.0501) (width 0.254) (layer "F.Cu") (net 8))
 (segment (start 149.31051 96.0501) (end 157.09851 103.8381) (width 0.254) (layer "F.Cu") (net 8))
 (segment (start 157.09851 103.8381) (end 157.77125 103.8381) (width 0.254) (layer "F.Cu") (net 8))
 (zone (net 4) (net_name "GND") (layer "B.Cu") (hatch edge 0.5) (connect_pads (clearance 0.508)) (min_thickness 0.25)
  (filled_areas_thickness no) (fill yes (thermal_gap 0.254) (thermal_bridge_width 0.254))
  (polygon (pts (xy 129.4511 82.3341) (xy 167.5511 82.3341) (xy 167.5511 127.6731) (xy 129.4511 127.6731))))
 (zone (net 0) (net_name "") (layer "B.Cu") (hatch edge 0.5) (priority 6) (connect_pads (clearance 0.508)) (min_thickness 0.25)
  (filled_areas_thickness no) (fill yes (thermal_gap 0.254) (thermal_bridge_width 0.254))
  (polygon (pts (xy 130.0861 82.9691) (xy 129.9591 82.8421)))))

